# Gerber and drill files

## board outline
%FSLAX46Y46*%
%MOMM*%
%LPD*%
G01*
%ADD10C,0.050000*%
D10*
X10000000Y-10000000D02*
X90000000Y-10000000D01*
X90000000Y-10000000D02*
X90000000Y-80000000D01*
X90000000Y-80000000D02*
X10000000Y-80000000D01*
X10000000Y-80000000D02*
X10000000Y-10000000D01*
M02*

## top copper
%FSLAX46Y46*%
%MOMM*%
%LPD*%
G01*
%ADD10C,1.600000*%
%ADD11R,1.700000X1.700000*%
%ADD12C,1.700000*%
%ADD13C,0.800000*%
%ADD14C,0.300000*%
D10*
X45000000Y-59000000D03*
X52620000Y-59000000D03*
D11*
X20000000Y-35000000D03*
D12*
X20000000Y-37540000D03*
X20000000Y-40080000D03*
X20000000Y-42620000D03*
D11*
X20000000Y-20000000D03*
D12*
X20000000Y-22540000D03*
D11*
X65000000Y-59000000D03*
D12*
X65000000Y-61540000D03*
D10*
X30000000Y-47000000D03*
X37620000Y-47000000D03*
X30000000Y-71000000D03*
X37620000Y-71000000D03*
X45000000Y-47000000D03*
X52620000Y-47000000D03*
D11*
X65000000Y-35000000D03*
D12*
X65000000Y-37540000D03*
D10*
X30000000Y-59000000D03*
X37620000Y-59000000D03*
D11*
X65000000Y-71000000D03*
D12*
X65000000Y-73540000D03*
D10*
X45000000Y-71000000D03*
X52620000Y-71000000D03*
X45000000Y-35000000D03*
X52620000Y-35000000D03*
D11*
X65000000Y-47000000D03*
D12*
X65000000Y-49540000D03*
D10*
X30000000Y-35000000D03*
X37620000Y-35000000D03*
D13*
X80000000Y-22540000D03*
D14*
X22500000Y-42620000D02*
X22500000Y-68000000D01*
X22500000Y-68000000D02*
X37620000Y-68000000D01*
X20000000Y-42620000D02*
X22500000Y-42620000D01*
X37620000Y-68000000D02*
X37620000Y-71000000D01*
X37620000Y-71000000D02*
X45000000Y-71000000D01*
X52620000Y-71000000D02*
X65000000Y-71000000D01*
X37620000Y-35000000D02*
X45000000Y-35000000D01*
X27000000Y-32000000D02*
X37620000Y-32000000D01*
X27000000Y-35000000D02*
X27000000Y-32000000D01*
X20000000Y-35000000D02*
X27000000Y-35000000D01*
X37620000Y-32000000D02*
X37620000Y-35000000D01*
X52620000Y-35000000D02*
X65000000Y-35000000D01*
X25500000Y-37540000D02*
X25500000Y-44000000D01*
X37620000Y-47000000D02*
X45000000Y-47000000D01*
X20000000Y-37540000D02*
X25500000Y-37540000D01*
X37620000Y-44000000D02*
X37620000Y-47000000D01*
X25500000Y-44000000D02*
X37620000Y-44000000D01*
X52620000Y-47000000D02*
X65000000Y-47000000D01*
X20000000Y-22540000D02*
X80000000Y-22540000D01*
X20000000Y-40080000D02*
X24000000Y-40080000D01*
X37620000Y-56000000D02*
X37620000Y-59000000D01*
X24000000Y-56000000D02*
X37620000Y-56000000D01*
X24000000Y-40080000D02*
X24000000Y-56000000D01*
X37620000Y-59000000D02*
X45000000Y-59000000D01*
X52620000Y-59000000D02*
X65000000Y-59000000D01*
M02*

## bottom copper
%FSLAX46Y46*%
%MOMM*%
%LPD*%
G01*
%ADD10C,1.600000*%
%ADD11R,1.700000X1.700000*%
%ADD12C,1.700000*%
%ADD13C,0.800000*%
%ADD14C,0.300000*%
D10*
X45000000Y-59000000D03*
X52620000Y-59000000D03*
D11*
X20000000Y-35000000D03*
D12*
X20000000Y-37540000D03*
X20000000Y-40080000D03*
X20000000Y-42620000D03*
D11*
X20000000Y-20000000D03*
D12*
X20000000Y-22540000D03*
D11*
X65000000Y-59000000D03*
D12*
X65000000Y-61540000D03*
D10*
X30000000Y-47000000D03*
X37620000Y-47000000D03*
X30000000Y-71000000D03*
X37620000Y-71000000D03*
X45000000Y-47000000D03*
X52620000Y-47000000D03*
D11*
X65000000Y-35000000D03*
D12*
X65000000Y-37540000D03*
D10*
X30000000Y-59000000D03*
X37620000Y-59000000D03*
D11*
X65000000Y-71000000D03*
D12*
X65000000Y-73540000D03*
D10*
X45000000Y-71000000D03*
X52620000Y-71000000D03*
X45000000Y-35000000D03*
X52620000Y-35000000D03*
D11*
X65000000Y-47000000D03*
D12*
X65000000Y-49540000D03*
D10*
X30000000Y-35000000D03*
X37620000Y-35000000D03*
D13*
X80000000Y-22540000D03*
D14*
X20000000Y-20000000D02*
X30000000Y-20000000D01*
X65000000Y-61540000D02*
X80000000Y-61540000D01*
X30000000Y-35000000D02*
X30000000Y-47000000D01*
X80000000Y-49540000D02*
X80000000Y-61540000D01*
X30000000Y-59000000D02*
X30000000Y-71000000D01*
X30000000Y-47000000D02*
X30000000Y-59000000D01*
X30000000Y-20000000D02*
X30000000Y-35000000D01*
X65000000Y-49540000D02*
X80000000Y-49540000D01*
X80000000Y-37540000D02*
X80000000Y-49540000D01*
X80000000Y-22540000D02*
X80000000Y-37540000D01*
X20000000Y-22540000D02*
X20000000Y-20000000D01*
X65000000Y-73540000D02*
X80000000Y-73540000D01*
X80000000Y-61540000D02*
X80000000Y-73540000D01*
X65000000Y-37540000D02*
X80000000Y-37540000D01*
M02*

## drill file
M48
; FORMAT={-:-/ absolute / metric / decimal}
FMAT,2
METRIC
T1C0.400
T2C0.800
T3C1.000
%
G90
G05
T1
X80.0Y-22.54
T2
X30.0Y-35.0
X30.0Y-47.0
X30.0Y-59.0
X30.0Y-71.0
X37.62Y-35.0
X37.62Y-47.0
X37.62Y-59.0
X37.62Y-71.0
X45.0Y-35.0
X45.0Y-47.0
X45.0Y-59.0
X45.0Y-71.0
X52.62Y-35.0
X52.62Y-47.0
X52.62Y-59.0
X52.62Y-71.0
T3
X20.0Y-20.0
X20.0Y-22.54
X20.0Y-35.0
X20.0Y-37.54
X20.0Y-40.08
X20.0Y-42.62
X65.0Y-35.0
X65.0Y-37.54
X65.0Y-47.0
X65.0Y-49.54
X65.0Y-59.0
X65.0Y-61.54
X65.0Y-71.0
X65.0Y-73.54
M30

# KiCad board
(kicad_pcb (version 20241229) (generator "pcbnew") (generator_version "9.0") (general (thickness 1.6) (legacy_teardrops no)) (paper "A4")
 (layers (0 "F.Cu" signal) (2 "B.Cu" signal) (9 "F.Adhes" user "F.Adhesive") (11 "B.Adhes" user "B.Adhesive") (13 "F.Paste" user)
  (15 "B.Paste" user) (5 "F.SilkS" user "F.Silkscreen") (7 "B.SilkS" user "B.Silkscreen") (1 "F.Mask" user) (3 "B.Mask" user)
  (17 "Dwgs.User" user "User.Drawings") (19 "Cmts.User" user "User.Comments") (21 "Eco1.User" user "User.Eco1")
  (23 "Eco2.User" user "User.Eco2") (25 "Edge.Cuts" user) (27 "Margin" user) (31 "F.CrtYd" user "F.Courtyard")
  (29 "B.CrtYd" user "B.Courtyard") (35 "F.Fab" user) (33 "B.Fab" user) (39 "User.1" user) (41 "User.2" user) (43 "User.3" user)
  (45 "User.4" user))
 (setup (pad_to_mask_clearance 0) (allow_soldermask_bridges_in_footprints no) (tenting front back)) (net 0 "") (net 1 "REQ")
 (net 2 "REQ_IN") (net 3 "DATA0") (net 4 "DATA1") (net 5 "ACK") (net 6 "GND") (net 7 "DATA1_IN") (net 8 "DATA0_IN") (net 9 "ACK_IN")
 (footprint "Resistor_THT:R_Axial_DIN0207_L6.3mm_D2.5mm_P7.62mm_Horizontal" (layer "F.Cu") (at 45 59)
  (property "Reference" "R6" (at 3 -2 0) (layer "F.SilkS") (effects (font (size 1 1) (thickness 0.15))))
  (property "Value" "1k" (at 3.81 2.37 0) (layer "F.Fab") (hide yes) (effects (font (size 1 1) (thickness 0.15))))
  (pad "1" thru_hole circle (at 0 0) (size 1.6 1.6) (drill 0.8) (layers "*.Cu" "*.Mask") (remove_unused_layers no) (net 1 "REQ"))
  (pad "2" thru_hole circle (at 7.62 0) (size 1.6 1.6) (drill 0.8) (layers "*.Cu" "*.Mask") (remove_unused_layers no) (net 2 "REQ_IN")))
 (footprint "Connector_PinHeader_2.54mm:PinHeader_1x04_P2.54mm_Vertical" (layer "F.Cu") (at 20 35)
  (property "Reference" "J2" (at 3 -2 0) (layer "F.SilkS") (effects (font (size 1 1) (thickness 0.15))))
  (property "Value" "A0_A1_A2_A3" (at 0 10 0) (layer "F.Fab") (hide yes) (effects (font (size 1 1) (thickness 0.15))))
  (pad "1" thru_hole rect (at 0 0) (size 1.7 1.7) (drill 1) (layers "*.Cu" "*.Mask") (remove_unused_layers no) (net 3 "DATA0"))
  (pad "2" thru_hole circle (at 0 2.54) (size 1.7 1.7) (drill 1) (layers "*.Cu" "*.Mask") (remove_unused_layers no) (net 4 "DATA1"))
  (pad "3" thru_hole circle (at 0 5.08) (size 1.7 1.7) (drill 1) (layers "*.Cu" "*.Mask") (remove_unused_layers no) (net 1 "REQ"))
  (pad "4" thru_hole circle (at 0 7.62) (size 1.7 1.7) (drill 1) (layers "*.Cu" "*.Mask") (remove_unused_layers no) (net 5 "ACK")))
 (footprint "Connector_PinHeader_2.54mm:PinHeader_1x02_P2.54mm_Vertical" (layer "F.Cu") (at 20 20)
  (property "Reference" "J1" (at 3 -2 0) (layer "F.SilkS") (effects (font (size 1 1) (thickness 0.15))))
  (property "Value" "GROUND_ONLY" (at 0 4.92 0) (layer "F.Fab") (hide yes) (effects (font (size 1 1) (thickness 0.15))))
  (pad "1" thru_hole rect (at 0 0) (size 1.7 1.7) (drill 1) (layers "*.Cu" "*.Mask") (remove_unused_layers no) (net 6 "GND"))
  (pad "2" thru_hole circle (at 0 2.54) (size 1.7 1.7) (drill 1) (layers "*.Cu" "*.Mask") (remove_unused_layers no) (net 6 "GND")))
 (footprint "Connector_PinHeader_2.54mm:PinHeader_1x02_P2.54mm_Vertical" (layer "F.Cu") (at 65 59)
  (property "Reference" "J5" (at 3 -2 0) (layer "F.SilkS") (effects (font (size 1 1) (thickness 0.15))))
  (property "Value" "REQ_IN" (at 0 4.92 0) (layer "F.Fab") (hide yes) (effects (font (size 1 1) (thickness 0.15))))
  (pad "1" thru_hole rect (at 0 0) (size 1.7 1.7) (drill 1) (layers "*.Cu" "*.Mask") (remove_unused_layers no) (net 2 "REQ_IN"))
  (pad "2" thru_hole circle (at 0 2.54) (size 1.7 1.7) (drill 1) (layers "*.Cu" "*.Mask") (remove_unused_layers no) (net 6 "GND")))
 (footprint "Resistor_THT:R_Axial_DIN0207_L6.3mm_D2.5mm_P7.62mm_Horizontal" (layer "F.Cu") (at 30 47)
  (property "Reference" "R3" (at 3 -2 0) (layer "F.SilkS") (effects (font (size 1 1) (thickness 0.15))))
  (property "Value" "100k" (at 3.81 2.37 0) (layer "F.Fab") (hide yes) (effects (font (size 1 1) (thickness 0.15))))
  (pad "1" thru_hole circle (at 0 0) (size 1.6 1.6) (drill 0.8) (layers "*.Cu" "*.Mask") (remove_unused_layers no) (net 6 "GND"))
  (pad "2" thru_hole circle (at 7.62 0) (size 1.6 1.6) (drill 0.8) (layers "*.Cu" "*.Mask") (remove_unused_layers no) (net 4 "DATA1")))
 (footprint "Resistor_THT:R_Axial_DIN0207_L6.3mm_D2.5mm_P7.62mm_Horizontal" (layer "F.Cu") (at 30 71)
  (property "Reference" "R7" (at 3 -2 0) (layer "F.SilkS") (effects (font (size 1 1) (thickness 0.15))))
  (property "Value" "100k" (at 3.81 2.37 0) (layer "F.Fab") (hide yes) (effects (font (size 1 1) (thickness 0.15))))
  (pad "1" thru_hole circle (at 0 0) (size 1.6 1.6) (drill 0.8) (layers "*.Cu" "*.Mask") (remove_unused_layers no) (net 6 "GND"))
  (pad "2" thru_hole circle (at 7.62 0) (size 1.6 1.6) (drill 0.8) (layers "*.Cu" "*.Mask") (remove_unused_layers no) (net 5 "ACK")))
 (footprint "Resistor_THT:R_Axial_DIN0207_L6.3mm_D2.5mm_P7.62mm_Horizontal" (layer "F.Cu") (at 45 47)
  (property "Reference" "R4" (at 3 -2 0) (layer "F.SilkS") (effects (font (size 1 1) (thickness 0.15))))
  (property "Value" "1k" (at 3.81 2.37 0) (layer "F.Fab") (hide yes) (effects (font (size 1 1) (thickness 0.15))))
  (pad "1" thru_hole circle (at 0 0) (size 1.6 1.6) (drill 0.8) (layers "*.Cu" "*.Mask") (remove_unused_layers no) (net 4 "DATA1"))
  (pad "2" thru_hole circle (at 7.62 0) (size 1.6 1.6) (drill 0.8) (layers "*.Cu" "*.Mask") (remove_unused_layers no) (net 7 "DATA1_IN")))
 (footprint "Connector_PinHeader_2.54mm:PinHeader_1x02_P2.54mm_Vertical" (layer "F.Cu") (at 65 35)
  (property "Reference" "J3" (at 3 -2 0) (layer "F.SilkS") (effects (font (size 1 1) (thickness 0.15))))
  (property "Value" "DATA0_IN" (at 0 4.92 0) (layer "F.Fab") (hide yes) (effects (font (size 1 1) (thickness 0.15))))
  (pad "1" thru_hole rect (at 0 0) (size 1.7 1.7) (drill 1) (layers "*.Cu" "*.Mask") (remove_unused_layers no) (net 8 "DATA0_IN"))
  (pad "2" thru_hole circle (at 0 2.54) (size 1.7 1.7) (drill 1) (layers "*.Cu" "*.Mask") (remove_unused_layers no) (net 6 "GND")))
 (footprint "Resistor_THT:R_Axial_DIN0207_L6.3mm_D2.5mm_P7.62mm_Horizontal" (layer "F.Cu") (at 30 59)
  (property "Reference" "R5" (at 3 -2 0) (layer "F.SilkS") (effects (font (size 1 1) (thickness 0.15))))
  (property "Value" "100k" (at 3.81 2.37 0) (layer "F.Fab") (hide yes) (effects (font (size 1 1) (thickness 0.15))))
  (pad "1" thru_hole circle (at 0 0) (size 1.6 1.6) (drill 0.8) (layers "*.Cu" "*.Mask") (remove_unused_layers no) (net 6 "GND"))
  (pad "2" thru_hole circle (at 7.62 0) (size 1.6 1.6) (drill 0.8) (layers "*.Cu" "*.Mask") (remove_unused_layers no) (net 1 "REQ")))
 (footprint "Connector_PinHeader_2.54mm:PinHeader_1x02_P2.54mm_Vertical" (layer "F.Cu") (at 65 71)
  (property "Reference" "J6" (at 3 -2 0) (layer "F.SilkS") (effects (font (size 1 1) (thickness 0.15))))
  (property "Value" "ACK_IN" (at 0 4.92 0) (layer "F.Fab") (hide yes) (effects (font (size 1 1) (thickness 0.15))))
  (pad "1" thru_hole rect (at 0 0) (size 1.7 1.7) (drill 1) (layers "*.Cu" "*.Mask") (remove_unused_layers no) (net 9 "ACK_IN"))
  (pad "2" thru_hole circle (at 0 2.54) (size 1.7 1.7) (drill 1) (layers "*.Cu" "*.Mask") (remove_unused_layers no) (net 6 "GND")))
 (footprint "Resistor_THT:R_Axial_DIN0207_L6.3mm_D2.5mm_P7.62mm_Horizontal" (layer "F.Cu") (at 45 71)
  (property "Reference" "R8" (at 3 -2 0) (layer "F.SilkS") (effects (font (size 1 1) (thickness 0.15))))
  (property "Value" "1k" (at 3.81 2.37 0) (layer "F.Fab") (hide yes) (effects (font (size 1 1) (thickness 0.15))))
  (pad "1" thru_hole circle (at 0 0) (size 1.6 1.6) (drill 0.8) (layers "*.Cu" "*.Mask") (remove_unused_layers no) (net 5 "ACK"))
  (pad "2" thru_hole circle (at 7.62 0) (size 1.6 1.6) (drill 0.8) (layers "*.Cu" "*.Mask") (remove_unused_layers no) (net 9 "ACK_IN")))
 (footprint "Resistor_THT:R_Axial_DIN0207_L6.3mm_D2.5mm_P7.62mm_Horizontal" (layer "F.Cu") (at 45 35)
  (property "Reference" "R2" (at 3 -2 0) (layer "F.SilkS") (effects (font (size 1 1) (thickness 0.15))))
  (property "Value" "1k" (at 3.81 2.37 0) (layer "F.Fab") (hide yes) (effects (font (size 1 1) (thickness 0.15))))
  (pad "1" thru_hole circle (at 0 0) (size 1.6 1.6) (drill 0.8) (layers "*.Cu" "*.Mask") (remove_unused_layers no) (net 3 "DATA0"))
  (pad "2" thru_hole circle (at 7.62 0) (size 1.6 1.6) (drill 0.8) (layers "*.Cu" "*.Mask") (remove_unused_layers no) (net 8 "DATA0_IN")))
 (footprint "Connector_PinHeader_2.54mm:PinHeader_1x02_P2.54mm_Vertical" (layer "F.Cu") (at 65 47)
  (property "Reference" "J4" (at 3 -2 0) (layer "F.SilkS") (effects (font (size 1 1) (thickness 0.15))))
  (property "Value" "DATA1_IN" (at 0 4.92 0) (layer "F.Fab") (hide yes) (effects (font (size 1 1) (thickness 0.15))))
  (pad "1" thru_hole rect (at 0 0) (size 1.7 1.7) (drill 1) (layers "*.Cu" "*.Mask") (remove_unused_layers no) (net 7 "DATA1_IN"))
  (pad "2" thru_hole circle (at 0 2.54) (size 1.7 1.7) (drill 1) (layers "*.Cu" "*.Mask") (remove_unused_layers no) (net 6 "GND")))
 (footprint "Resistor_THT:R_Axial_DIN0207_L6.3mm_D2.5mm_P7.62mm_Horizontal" (layer "F.Cu") (at 30 35)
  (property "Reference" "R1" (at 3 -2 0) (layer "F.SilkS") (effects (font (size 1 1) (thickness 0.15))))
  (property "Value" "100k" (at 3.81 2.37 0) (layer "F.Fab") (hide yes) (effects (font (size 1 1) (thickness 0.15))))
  (pad "1" thru_hole circle (at 0 0) (size 1.6 1.6) (drill 0.8) (layers "*.Cu" "*.Mask") (remove_unused_layers no) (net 6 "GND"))
  (pad "2" thru_hole circle (at 7.62 0) (size 1.6 1.6) (drill 0.8) (layers "*.Cu" "*.Mask") (remove_unused_layers no) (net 3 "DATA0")))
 (gr_line (start 10 10) (end 90 10) (stroke (width 0.05) (type default)) (layer "Edge.Cuts"))
 (gr_line (start 90 10) (end 90 80) (stroke (width 0.05) (type default)) (layer "Edge.Cuts"))
 (gr_line (start 90 80) (end 10 80) (stroke (width 0.05) (type default)) (layer "Edge.Cuts"))
 (gr_line (start 10 80) (end 10 10) (stroke (width 0.05) (type default)) (layer "Edge.Cuts"))
 (segment (start 22.5 42.62) (end 22.5 68) (width 0.3) (layer "F.Cu") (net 5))
 (segment (start 22.5 68) (end 37.62 68) (width 0.3) (layer "F.Cu") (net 5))
 (segment (start 20 42.62) (end 22.5 42.62) (width 0.3) (layer "F.Cu") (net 5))
 (segment (start 37.62 68) (end 37.62 71) (width 0.3) (layer "F.Cu") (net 5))
 (segment (start 37.62 71) (end 45 71) (width 0.3) (layer "F.Cu") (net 5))
 (segment (start 52.62 71) (end 65 71) (width 0.3) (layer "F.Cu") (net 9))
 (segment (start 37.62 35) (end 45 35) (width 0.3) (layer "F.Cu") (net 3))
 (segment (start 27 32) (end 37.62 32) (width 0.3) (layer "F.Cu") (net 3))
 (segment (start 27 35) (end 27 32) (width 0.3) (layer "F.Cu") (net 3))
 (segment (start 20 35) (end 27 35) (width 0.3) (layer "F.Cu") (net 3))
 (segment (start 37.62 32) (end 37.62 35) (width 0.3) (layer "F.Cu") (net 3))
 (segment (start 52.62 35) (end 65 35) (width 0.3) (layer "F.Cu") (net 8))
 (segment (start 25.5 37.54) (end 25.5 44) (width 0.3) (layer "F.Cu") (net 4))
 (segment (start 37.62 47) (end 45 47) (width 0.3) (layer "F.Cu") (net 4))
 (segment (start 20 37.54) (end 25.5 37.54) (width 0.3) (layer "F.Cu") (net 4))
 (segment (start 37.62 44) (end 37.62 47) (width 0.3) (layer "F.Cu") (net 4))
 (segment (start 25.5 44) (end 37.62 44) (width 0.3) (layer "F.Cu") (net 4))
 (segment (start 52.62 47) (end 65 47) (width 0.3) (layer "F.Cu") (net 7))
 (segment (start 20 22.54) (end 80 22.54) (width 0.3) (layer "F.Cu") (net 6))
 (via (at 80 22.54) (size 0.8) (drill 0.4) (layers "F.Cu" "B.Cu") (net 6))
 (segment (start 20 20) (end 30 20) (width 0.3) (layer "B.Cu") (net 6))
 (segment (start 65 61.54) (end 80 61.54) (width 0.3) (layer "B.Cu") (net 6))
 (segment (start 30 35) (end 30 47) (width 0.3) (layer "B.Cu") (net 6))
 (segment (start 80 49.54) (end 80 61.54) (width 0.3) (layer "B.Cu") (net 6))
 (segment (start 30 59) (end 30 71) (width 0.3) (layer "B.Cu") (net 6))
 (segment (start 30 47) (end 30 59) (width 0.3) (layer "B.Cu") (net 6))
 (segment (start 30 20) (end 30 35) (width 0.3) (layer "B.Cu") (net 6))
 (segment (start 65 49.54) (end 80 49.54) (width 0.3) (layer "B.Cu") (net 6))
 (segment (start 80 37.54) (end 80 49.54) (width 0.3) (layer "B.Cu") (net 6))
 (segment (start 80 22.54) (end 80 37.54) (width 0.3) (layer "B.Cu") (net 6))
 (segment (start 20 22.54) (end 20 20) (width 0.3) (layer "B.Cu") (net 6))
 (segment (start 65 73.54) (end 80 73.54) (width 0.3) (layer "B.Cu") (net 6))
 (segment (start 80 61.54) (end 80 73.54) (width 0.3) (layer "B.Cu") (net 6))
 (segment (start 65 37.54) (end 80 37.54) (width 0.3) (layer "B.Cu") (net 6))
 (segment (start 20 40.08) (end 24 40.08) (width 0.3) (layer "F.Cu") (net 1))
 (segment (start 37.62 56) (end 37.62 59) (width 0.3) (layer "F.Cu") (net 1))
 (segment (start 24 56) (end 37.62 56) (width 0.3) (layer "F.Cu") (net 1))
 (segment (start 24 40.08) (end 24 56) (width 0.3) (layer "F.Cu") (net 1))
 (segment (start 37.62 59) (end 45 59) (width 0.3) (layer "F.Cu") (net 1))
 (segment (start 52.62 59) (end 65 59) (width 0.3) (layer "F.Cu") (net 2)))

